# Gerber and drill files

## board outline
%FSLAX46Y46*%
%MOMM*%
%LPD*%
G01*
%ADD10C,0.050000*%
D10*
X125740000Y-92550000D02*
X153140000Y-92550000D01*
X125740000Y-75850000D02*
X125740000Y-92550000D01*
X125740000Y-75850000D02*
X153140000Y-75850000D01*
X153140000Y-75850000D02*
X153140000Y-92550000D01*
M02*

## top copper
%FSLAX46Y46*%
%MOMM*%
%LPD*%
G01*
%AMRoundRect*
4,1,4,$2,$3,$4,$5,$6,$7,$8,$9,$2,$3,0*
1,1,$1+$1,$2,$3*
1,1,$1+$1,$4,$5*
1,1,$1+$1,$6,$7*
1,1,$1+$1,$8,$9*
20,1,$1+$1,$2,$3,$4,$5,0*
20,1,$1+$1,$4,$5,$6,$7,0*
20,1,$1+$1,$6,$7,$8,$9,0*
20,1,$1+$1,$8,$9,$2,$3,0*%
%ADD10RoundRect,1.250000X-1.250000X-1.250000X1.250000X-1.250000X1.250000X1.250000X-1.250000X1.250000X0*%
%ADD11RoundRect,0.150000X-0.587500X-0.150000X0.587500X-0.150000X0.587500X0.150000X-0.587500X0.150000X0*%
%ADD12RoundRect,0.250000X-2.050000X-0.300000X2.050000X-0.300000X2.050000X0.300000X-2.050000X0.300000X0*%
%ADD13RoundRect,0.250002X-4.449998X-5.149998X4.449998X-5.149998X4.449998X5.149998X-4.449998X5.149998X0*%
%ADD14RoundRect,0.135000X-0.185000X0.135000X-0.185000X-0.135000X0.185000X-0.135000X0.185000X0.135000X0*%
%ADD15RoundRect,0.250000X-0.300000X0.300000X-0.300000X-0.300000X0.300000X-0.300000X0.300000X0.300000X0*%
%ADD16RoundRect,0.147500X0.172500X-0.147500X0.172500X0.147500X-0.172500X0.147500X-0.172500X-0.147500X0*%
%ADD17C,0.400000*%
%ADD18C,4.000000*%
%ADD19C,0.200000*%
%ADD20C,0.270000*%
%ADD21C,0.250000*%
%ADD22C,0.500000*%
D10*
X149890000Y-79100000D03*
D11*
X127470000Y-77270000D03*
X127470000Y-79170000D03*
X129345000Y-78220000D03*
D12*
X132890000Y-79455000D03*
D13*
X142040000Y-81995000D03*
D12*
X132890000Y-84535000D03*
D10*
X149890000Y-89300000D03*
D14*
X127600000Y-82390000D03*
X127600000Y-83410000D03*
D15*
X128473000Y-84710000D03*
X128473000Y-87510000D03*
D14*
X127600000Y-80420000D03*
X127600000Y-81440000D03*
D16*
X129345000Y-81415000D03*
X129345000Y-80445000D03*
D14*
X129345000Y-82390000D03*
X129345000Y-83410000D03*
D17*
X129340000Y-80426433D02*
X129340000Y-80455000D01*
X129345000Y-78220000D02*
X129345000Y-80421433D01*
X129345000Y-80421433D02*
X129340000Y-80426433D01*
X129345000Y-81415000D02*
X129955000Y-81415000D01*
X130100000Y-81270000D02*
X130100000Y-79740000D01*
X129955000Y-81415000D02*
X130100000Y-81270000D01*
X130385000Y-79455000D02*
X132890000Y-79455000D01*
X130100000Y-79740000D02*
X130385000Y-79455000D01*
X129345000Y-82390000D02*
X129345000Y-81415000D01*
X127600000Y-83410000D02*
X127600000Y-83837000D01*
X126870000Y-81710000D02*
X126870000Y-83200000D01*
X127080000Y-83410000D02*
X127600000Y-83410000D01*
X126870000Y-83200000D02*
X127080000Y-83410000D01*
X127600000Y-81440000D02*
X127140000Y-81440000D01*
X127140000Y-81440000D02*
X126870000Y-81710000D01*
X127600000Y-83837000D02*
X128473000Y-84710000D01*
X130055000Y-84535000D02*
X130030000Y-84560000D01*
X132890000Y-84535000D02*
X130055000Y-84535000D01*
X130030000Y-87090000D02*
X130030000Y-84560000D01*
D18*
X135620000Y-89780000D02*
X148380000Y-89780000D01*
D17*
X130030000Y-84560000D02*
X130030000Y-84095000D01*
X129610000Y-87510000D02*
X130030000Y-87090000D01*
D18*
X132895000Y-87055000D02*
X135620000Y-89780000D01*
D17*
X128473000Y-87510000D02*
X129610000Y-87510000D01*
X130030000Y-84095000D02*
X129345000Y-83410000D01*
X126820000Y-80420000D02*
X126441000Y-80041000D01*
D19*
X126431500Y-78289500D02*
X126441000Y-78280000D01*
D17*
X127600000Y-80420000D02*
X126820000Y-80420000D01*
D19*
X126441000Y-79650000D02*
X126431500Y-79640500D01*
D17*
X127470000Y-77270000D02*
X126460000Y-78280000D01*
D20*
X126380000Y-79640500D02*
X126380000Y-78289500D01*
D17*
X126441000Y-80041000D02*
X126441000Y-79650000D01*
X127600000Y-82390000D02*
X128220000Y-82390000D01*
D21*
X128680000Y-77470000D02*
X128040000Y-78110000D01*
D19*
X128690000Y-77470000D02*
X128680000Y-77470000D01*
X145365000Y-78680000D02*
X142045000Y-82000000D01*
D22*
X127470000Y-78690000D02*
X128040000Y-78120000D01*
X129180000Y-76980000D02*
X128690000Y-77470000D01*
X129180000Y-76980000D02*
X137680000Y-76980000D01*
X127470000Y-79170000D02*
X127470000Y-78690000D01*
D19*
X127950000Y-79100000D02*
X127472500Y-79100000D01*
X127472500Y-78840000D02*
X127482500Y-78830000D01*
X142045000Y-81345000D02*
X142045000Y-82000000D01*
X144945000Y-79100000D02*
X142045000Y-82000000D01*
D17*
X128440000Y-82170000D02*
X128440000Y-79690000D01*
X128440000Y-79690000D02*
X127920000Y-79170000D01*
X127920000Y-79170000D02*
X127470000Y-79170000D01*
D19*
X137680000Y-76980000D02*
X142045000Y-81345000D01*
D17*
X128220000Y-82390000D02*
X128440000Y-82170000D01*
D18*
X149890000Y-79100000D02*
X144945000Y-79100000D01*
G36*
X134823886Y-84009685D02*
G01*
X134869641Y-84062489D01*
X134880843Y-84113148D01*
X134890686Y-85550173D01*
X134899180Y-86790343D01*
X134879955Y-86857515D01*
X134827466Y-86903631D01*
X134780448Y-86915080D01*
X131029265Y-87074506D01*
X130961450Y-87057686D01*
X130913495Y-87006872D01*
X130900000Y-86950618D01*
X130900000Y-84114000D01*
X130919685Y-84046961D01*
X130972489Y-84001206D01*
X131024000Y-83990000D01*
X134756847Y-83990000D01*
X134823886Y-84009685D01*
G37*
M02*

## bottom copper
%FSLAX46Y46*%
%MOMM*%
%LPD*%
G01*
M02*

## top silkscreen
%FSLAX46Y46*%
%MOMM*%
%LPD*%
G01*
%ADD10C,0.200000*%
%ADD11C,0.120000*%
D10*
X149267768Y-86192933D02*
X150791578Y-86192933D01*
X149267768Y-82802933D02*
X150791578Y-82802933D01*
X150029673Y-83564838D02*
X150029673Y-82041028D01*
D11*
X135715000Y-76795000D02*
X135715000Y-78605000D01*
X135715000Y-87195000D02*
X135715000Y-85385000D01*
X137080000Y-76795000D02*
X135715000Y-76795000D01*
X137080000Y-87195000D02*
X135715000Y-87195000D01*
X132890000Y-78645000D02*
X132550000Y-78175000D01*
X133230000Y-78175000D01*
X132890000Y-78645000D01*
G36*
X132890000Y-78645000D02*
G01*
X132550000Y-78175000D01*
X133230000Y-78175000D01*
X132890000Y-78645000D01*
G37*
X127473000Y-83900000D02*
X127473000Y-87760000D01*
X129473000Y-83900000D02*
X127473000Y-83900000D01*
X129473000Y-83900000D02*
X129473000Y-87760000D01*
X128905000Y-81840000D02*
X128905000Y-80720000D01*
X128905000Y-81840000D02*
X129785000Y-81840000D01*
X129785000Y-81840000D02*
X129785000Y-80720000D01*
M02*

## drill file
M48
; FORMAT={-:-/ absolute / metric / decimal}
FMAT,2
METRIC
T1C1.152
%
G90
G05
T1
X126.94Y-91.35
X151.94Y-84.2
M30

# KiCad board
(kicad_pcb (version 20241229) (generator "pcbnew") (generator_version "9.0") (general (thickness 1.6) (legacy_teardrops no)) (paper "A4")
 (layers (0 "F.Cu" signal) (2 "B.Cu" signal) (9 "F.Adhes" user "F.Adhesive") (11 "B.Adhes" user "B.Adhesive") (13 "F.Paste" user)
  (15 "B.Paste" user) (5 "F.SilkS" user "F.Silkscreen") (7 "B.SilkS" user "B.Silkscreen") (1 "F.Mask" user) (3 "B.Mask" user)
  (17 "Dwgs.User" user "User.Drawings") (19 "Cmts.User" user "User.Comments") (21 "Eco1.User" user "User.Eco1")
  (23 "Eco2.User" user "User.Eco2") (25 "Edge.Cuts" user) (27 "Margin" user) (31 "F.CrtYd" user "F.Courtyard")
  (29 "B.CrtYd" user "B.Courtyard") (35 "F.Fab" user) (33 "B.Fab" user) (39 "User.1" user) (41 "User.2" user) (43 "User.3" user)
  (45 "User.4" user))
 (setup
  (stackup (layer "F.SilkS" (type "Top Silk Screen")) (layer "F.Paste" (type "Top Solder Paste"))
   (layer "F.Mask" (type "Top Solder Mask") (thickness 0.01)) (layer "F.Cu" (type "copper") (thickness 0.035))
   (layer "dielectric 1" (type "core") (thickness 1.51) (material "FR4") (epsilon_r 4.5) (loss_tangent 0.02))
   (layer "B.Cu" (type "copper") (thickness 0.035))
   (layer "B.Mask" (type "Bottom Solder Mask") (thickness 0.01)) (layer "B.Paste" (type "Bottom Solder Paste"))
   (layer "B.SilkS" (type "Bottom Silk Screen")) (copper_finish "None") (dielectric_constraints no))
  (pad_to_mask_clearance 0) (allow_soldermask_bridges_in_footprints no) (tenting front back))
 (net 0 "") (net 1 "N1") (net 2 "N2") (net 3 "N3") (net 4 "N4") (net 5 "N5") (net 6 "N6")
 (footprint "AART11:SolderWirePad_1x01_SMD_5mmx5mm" (layer "F.Cu") (at 149.89 79.1)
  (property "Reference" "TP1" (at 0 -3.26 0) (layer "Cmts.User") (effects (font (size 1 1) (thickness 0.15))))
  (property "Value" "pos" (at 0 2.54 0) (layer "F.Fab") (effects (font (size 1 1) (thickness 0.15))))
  (pad "1" smd roundrect (at 0 0) (size 5 5) (layers "F.Cu" "F.Mask" "F.Paste") (roundrect_rratio 0.25) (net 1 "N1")))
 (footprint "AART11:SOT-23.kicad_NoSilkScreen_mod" (layer "F.Cu") (at 128.4075 78.22)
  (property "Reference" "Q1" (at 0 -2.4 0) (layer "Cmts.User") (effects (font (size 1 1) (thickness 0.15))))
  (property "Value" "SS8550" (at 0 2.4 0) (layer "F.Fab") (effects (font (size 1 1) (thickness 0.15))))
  (pad "1" smd roundrect (at -0.9375 -0.95) (size 1.475 0.6) (layers "F.Cu" "F.Mask" "F.Paste") (roundrect_rratio 0.25) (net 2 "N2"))
  (pad "2" smd roundrect (at -0.9375 0.95) (size 1.475 0.6) (layers "F.Cu" "F.Mask" "F.Paste") (roundrect_rratio 0.25) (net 1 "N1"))
  (pad "3" smd roundrect (at 0.9375 0) (size 1.475 0.6) (layers "F.Cu" "F.Mask" "F.Paste") (roundrect_rratio 0.25) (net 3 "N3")))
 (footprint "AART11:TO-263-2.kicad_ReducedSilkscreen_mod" (layer "F.Cu") (at 140.54 81.995)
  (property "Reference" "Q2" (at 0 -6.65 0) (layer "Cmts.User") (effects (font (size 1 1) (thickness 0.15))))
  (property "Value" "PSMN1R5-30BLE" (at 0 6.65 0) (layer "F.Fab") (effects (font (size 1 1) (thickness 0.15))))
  (fp_line (start -4.825 -5.2) (end -4.825 -3.39) (stroke (width 0.12) (type solid)) (layer "F.SilkS"))
  (fp_line (start -4.825 5.2) (end -4.825 3.39) (stroke (width 0.12) (type solid)) (layer "F.SilkS"))
  (fp_line (start -3.46 -5.2) (end -4.825 -5.2) (stroke (width 0.12) (type solid)) (layer "F.SilkS"))
  (fp_line (start -3.46 5.2) (end -4.825 5.2) (stroke (width 0.12) (type solid)) (layer "F.SilkS"))
  (fp_poly (pts (xy -7.65 -3.35) (xy -7.99 -3.82) (xy -7.31 -3.82)) (stroke (width 0.12) (type solid)) (fill yes) (layer "F.SilkS"))
  (pad "" smd roundrect (at -0.925 -2.775) (size 4.55 5.25) (layers "F.Paste") (roundrect_rratio 0.054945))
  (pad "" smd roundrect (at -0.925 2.775) (size 4.55 5.25) (layers "F.Paste") (roundrect_rratio 0.054945))
  (pad "" smd roundrect (at 3.925 -2.775) (size 4.55 5.25) (layers "F.Paste") (roundrect_rratio 0.054945))
  (pad "" smd roundrect (at 3.925 2.775) (size 4.55 5.25) (layers "F.Paste") (roundrect_rratio 0.054945))
  (pad "1" smd roundrect (at -7.65 -2.54) (size 4.6 1.1) (layers "F.Cu" "F.Mask" "F.Paste") (roundrect_rratio 0.227273) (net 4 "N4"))
  (pad "2" smd roundrect (at 1.5 0) (size 9.4 10.8) (layers "F.Cu" "F.Mask") (roundrect_rratio 0.026596) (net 1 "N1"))
  (pad "3" smd roundrect (at -7.65 2.54) (size 4.6 1.1) (layers "F.Cu" "F.Mask" "F.Paste") (roundrect_rratio 0.227273) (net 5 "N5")))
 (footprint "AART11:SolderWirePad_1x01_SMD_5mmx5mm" (layer "F.Cu") (at 149.89 89.3)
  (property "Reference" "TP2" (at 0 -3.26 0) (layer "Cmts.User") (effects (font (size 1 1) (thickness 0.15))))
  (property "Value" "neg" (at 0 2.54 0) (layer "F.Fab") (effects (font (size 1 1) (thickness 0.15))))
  (pad "1" smd roundrect (at 0 0) (size 5 5) (layers "F.Cu" "F.Mask" "F.Paste") (roundrect_rratio 0.25) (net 5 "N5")))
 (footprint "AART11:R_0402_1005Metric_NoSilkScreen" (layer "F.Cu") (at 127.6 82.9 -90)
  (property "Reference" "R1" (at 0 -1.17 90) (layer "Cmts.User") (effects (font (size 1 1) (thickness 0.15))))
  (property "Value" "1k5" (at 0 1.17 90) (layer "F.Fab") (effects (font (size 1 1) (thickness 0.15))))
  (pad "1" smd roundrect (at -0.51 0 270) (size 0.54 0.64) (layers "F.Cu" "F.Mask" "F.Paste") (roundrect_rratio 0.25) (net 1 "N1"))
  (pad "2" smd roundrect (at 0.51 0 270) (size 0.54 0.64) (layers "F.Cu" "F.Mask" "F.Paste") (roundrect_rratio 0.25) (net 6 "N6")))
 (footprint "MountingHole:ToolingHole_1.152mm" (layer "F.Cu") (at 151.94 84.2)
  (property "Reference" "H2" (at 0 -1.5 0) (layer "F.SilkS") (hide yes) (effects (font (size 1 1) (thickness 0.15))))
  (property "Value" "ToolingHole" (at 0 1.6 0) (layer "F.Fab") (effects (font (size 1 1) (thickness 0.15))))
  (pad "" np_thru_hole circle (at 0 0) (size 1.152 1.152) (drill 1.152) (layers "*.Cu" "*.Mask") (solder_mask_margin 0.074))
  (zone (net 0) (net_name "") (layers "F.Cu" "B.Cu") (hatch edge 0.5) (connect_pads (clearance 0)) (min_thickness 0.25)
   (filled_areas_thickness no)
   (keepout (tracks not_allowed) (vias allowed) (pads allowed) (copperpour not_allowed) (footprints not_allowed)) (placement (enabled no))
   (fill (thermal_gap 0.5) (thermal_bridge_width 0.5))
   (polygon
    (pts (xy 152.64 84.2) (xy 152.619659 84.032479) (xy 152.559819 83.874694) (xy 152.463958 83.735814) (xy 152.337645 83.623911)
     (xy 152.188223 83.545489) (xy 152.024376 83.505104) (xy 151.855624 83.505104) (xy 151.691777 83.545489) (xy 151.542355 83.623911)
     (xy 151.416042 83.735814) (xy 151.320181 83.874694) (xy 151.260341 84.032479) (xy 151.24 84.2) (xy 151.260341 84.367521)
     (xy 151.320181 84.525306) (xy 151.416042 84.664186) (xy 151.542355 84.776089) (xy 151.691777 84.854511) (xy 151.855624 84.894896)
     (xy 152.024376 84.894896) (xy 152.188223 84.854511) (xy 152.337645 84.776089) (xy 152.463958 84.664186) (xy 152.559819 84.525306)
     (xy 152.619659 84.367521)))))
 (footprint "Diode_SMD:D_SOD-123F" (layer "F.Cu") (at 128.473 86.11 -90)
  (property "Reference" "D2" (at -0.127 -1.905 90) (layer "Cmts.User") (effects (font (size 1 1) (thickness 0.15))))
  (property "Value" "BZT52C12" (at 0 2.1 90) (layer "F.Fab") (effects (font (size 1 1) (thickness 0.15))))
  (fp_line (start -2.21 1) (end 1.65 1) (stroke (width 0.12) (type solid)) (layer "F.SilkS"))
  (fp_line (start -2.21 -1) (end -2.21 1) (stroke (width 0.12) (type solid)) (layer "F.SilkS"))
  (fp_line (start -2.21 -1) (end 1.65 -1) (stroke (width 0.12) (type solid)) (layer "F.SilkS"))
  (pad "1" smd roundrect (at -1.4 0 270) (size 1.1 1.1) (layers "F.Cu" "F.Mask" "F.Paste") (roundrect_rratio 0.2272727273) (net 6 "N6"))
  (pad "2" smd roundrect (at 1.4 0 270) (size 1.1 1.1) (layers "F.Cu" "F.Mask" "F.Paste") (roundrect_rratio 0.2272727273) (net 5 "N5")))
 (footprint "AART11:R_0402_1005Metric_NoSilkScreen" (layer "F.Cu") (at 127.6 80.93 -90)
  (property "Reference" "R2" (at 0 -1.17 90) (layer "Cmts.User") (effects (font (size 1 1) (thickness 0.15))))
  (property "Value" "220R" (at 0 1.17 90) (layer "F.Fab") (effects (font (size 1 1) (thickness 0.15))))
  (pad "1" smd roundrect (at -0.51 0 270) (size 0.54 0.64) (layers "F.Cu" "F.Mask" "F.Paste") (roundrect_rratio 0.25) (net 2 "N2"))
  (pad "2" smd roundrect (at 0.51 0 270) (size 0.54 0.64) (layers "F.Cu" "F.Mask" "F.Paste") (roundrect_rratio 0.25) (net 6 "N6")))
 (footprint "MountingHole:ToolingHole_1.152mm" (layer "F.Cu") (at 126.94 91.35)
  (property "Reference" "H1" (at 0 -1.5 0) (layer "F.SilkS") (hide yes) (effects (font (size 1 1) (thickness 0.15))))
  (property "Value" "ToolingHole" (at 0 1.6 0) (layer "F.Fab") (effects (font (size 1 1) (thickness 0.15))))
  (pad "" np_thru_hole circle (at 0 0) (size 1.152 1.152) (drill 1.152) (layers "*.Cu" "*.Mask") (solder_mask_margin 0.074))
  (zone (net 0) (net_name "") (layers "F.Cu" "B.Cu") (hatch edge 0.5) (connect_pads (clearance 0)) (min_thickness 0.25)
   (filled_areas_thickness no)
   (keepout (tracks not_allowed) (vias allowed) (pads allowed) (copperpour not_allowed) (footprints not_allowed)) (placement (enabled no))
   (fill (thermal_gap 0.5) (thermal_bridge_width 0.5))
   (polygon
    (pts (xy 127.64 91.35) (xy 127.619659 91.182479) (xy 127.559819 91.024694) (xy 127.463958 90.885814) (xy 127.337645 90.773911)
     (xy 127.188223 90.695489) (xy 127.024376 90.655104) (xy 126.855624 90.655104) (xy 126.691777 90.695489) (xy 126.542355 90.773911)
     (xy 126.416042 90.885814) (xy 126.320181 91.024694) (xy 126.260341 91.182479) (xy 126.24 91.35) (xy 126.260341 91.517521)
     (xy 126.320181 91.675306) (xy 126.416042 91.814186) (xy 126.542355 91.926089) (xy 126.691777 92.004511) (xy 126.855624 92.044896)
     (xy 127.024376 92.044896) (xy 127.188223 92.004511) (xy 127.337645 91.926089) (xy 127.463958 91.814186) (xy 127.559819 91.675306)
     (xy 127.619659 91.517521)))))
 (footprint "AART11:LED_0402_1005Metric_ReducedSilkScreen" (layer "F.Cu") (at 129.345 80.93 90)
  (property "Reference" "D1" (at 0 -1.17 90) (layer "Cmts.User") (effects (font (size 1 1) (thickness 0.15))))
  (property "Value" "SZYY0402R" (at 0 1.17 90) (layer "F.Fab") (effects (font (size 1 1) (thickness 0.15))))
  (fp_line (start -0.91 -0.44) (end 0.21 -0.44) (stroke (width 0.12) (type default)) (layer "F.SilkS"))
  (fp_line (start -0.91 -0.44) (end -0.91 0.44) (stroke (width 0.12) (type default)) (layer "F.SilkS"))
  (fp_line (start -0.91 0.44) (end 0.21 0.44) (stroke (width 0.12) (type default)) (layer "F.SilkS"))
  (pad "1" smd roundrect (at -0.485 0 90) (size 0.59 0.64) (layers "F.Cu" "F.Mask" "F.Paste") (roundrect_rratio 0.25) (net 4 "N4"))
  (pad "2" smd roundrect (at 0.485 0 90) (size 0.59 0.64) (layers "F.Cu" "F.Mask" "F.Paste") (roundrect_rratio 0.25) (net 3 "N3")))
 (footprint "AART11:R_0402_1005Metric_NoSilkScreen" (layer "F.Cu") (at 129.345 82.9 -90)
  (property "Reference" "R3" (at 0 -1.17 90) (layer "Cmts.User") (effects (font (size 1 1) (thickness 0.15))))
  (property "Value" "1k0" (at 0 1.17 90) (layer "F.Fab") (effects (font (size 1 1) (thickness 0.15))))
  (pad "1" smd roundrect (at -0.51 0 270) (size 0.54 0.64) (layers "F.Cu" "F.Mask" "F.Paste") (roundrect_rratio 0.25) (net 4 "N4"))
  (pad "2" smd roundrect (at 0.51 0 270) (size 0.54 0.64) (layers "F.Cu" "F.Mask" "F.Paste") (roundrect_rratio 0.25) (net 5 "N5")))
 (gr_line (start 125.74 92.55) (end 153.14 92.55) (stroke (width 0.05) (type solid)) (layer "Edge.Cuts"))
 (gr_line (start 125.74 75.85) (end 125.74 92.55) (stroke (width 0.05) (type solid)) (layer "Edge.Cuts"))
 (gr_line (start 125.74 75.85) (end 153.14 75.85) (stroke (width 0.05) (type solid)) (layer "Edge.Cuts"))
 (gr_line (start 153.14 75.85) (end 153.14 92.55) (stroke (width 0.05) (type solid)) (layer "Edge.Cuts"))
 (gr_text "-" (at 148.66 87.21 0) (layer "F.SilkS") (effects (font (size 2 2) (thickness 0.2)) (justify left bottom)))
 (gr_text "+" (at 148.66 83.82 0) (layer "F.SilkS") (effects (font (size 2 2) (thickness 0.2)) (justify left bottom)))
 (segment (start 129.34 80.426433) (end 129.34 80.455) (width 0.4) (layer "F.Cu") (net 3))
 (segment (start 129.345 78.22) (end 129.345 80.421433) (width 0.4) (layer "F.Cu") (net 3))
 (segment (start 129.345 80.421433) (end 129.34 80.426433) (width 0.4) (layer "F.Cu") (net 3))
 (segment (start 129.345 81.415) (end 129.955 81.415) (width 0.4) (layer "F.Cu") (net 4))
 (segment (start 130.1 81.27) (end 130.1 79.74) (width 0.4) (layer "F.Cu") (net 4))
 (segment (start 129.955 81.415) (end 130.1 81.27) (width 0.4) (layer "F.Cu") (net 4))
 (segment (start 130.385 79.455) (end 132.89 79.455) (width 0.4) (layer "F.Cu") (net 4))
 (segment (start 130.1 79.74) (end 130.385 79.455) (width 0.4) (layer "F.Cu") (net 4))
 (segment (start 129.345 82.39) (end 129.345 81.415) (width 0.4) (layer "F.Cu") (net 4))
 (segment (start 127.6 83.41) (end 127.6 83.837) (width 0.4) (layer "F.Cu") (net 6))
 (segment (start 126.87 81.71) (end 126.87 83.2) (width 0.4) (layer "F.Cu") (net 6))
 (segment (start 127.08 83.41) (end 127.6 83.41) (width 0.4) (layer "F.Cu") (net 6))
 (segment (start 126.87 83.2) (end 127.08 83.41) (width 0.4) (layer "F.Cu") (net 6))
 (segment (start 127.6 81.44) (end 127.14 81.44) (width 0.4) (layer "F.Cu") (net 6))
 (segment (start 127.14 81.44) (end 126.87 81.71) (width 0.4) (layer "F.Cu") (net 6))
 (segment (start 127.6 83.837) (end 128.473 84.71) (width 0.4) (layer "F.Cu") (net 6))
 (segment (start 130.055 84.535) (end 130.03 84.56) (width 0.4) (layer "F.Cu") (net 5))
 (segment (start 132.89 84.535) (end 130.055 84.535) (width 0.4) (layer "F.Cu") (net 5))
 (segment (start 130.03 87.09) (end 130.03 84.56) (width 0.4) (layer "F.Cu") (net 5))
 (segment (start 135.62 89.78) (end 148.38 89.78) (width 4) (layer "F.Cu") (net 5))
 (segment (start 130.03 84.56) (end 130.03 84.095) (width 0.4) (layer "F.Cu") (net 5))
 (segment (start 129.61 87.51) (end 130.03 87.09) (width 0.4) (layer "F.Cu") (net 5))
 (segment (start 132.895 87.055) (end 135.62 89.78) (width 4) (layer "F.Cu") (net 5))
 (segment (start 128.473 87.51) (end 129.61 87.51) (width 0.4) (layer "F.Cu") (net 5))
 (segment (start 130.03 84.095) (end 129.345 83.41) (width 0.4) (layer "F.Cu") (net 5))
 (segment (start 126.82 80.42) (end 126.441 80.041) (width 0.4) (layer "F.Cu") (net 2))
 (segment (start 126.4315 78.2895) (end 126.441 78.28) (width 0.2) (layer "F.Cu") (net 2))
 (segment (start 127.6 80.42) (end 126.82 80.42) (width 0.4) (layer "F.Cu") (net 2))
 (segment (start 126.441 79.65) (end 126.4315 79.6405) (width 0.2) (layer "F.Cu") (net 2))
 (segment (start 127.47 77.27) (end 126.46 78.28) (width 0.4) (layer "F.Cu") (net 2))
 (segment (start 126.38 79.6405) (end 126.38 78.2895) (width 0.27) (layer "F.Cu") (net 2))
 (segment (start 126.441 80.041) (end 126.441 79.65) (width 0.4) (layer "F.Cu") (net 2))
 (segment (start 127.6 82.39) (end 128.22 82.39) (width 0.4) (layer "F.Cu") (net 1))
 (segment (start 128.68 77.47) (end 128.04 78.11) (width 0.25) (layer "F.Cu") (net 1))
 (segment (start 128.69 77.47) (end 128.68 77.47) (width 0.2) (layer "F.Cu") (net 1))
 (segment (start 145.365 78.68) (end 142.045 82) (width 0.2) (layer "F.Cu") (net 1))
 (segment (start 127.47 78.69) (end 128.04 78.12) (width 0.5) (layer "F.Cu") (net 1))
 (segment (start 129.18 76.98) (end 128.69 77.47) (width 0.5) (layer "F.Cu") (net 1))
 (segment (start 129.18 76.98) (end 137.68 76.98) (width 0.5) (layer "F.Cu") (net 1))
 (segment (start 127.47 79.17) (end 127.47 78.69) (width 0.5) (layer "F.Cu") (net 1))
 (segment (start 127.95 79.1) (end 127.4725 79.1) (width 0.2) (layer "F.Cu") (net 1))
 (segment (start 127.4725 78.84) (end 127.4825 78.83) (width 0.2) (layer "F.Cu") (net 1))
 (segment (start 142.045 81.345) (end 142.045 82) (width 0.2) (layer "F.Cu") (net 1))
 (segment (start 144.945 79.1) (end 142.045 82) (width 0.2) (layer "F.Cu") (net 1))
 (segment (start 128.44 82.17) (end 128.44 79.69) (width 0.4) (layer "F.Cu") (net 1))
 (segment (start 128.44 79.69) (end 127.92 79.17) (width 0.4) (layer "F.Cu") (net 1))
 (segment (start 127.92 79.17) (end 127.47 79.17) (width 0.4) (layer "F.Cu") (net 1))
 (segment (start 137.68 76.98) (end 142.045 81.345) (width 0.2) (layer "F.Cu") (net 1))
 (segment (start 128.22 82.39) (end 128.44 82.17) (width 0.4) (layer "F.Cu") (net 1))
 (segment (start 149.89 79.1) (end 144.945 79.1) (width 4) (layer "F.Cu") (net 1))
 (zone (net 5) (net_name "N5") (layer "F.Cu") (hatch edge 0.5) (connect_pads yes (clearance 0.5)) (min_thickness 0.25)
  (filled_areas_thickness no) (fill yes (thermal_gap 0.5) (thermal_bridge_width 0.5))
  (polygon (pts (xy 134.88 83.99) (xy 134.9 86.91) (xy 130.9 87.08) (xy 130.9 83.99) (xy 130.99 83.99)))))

